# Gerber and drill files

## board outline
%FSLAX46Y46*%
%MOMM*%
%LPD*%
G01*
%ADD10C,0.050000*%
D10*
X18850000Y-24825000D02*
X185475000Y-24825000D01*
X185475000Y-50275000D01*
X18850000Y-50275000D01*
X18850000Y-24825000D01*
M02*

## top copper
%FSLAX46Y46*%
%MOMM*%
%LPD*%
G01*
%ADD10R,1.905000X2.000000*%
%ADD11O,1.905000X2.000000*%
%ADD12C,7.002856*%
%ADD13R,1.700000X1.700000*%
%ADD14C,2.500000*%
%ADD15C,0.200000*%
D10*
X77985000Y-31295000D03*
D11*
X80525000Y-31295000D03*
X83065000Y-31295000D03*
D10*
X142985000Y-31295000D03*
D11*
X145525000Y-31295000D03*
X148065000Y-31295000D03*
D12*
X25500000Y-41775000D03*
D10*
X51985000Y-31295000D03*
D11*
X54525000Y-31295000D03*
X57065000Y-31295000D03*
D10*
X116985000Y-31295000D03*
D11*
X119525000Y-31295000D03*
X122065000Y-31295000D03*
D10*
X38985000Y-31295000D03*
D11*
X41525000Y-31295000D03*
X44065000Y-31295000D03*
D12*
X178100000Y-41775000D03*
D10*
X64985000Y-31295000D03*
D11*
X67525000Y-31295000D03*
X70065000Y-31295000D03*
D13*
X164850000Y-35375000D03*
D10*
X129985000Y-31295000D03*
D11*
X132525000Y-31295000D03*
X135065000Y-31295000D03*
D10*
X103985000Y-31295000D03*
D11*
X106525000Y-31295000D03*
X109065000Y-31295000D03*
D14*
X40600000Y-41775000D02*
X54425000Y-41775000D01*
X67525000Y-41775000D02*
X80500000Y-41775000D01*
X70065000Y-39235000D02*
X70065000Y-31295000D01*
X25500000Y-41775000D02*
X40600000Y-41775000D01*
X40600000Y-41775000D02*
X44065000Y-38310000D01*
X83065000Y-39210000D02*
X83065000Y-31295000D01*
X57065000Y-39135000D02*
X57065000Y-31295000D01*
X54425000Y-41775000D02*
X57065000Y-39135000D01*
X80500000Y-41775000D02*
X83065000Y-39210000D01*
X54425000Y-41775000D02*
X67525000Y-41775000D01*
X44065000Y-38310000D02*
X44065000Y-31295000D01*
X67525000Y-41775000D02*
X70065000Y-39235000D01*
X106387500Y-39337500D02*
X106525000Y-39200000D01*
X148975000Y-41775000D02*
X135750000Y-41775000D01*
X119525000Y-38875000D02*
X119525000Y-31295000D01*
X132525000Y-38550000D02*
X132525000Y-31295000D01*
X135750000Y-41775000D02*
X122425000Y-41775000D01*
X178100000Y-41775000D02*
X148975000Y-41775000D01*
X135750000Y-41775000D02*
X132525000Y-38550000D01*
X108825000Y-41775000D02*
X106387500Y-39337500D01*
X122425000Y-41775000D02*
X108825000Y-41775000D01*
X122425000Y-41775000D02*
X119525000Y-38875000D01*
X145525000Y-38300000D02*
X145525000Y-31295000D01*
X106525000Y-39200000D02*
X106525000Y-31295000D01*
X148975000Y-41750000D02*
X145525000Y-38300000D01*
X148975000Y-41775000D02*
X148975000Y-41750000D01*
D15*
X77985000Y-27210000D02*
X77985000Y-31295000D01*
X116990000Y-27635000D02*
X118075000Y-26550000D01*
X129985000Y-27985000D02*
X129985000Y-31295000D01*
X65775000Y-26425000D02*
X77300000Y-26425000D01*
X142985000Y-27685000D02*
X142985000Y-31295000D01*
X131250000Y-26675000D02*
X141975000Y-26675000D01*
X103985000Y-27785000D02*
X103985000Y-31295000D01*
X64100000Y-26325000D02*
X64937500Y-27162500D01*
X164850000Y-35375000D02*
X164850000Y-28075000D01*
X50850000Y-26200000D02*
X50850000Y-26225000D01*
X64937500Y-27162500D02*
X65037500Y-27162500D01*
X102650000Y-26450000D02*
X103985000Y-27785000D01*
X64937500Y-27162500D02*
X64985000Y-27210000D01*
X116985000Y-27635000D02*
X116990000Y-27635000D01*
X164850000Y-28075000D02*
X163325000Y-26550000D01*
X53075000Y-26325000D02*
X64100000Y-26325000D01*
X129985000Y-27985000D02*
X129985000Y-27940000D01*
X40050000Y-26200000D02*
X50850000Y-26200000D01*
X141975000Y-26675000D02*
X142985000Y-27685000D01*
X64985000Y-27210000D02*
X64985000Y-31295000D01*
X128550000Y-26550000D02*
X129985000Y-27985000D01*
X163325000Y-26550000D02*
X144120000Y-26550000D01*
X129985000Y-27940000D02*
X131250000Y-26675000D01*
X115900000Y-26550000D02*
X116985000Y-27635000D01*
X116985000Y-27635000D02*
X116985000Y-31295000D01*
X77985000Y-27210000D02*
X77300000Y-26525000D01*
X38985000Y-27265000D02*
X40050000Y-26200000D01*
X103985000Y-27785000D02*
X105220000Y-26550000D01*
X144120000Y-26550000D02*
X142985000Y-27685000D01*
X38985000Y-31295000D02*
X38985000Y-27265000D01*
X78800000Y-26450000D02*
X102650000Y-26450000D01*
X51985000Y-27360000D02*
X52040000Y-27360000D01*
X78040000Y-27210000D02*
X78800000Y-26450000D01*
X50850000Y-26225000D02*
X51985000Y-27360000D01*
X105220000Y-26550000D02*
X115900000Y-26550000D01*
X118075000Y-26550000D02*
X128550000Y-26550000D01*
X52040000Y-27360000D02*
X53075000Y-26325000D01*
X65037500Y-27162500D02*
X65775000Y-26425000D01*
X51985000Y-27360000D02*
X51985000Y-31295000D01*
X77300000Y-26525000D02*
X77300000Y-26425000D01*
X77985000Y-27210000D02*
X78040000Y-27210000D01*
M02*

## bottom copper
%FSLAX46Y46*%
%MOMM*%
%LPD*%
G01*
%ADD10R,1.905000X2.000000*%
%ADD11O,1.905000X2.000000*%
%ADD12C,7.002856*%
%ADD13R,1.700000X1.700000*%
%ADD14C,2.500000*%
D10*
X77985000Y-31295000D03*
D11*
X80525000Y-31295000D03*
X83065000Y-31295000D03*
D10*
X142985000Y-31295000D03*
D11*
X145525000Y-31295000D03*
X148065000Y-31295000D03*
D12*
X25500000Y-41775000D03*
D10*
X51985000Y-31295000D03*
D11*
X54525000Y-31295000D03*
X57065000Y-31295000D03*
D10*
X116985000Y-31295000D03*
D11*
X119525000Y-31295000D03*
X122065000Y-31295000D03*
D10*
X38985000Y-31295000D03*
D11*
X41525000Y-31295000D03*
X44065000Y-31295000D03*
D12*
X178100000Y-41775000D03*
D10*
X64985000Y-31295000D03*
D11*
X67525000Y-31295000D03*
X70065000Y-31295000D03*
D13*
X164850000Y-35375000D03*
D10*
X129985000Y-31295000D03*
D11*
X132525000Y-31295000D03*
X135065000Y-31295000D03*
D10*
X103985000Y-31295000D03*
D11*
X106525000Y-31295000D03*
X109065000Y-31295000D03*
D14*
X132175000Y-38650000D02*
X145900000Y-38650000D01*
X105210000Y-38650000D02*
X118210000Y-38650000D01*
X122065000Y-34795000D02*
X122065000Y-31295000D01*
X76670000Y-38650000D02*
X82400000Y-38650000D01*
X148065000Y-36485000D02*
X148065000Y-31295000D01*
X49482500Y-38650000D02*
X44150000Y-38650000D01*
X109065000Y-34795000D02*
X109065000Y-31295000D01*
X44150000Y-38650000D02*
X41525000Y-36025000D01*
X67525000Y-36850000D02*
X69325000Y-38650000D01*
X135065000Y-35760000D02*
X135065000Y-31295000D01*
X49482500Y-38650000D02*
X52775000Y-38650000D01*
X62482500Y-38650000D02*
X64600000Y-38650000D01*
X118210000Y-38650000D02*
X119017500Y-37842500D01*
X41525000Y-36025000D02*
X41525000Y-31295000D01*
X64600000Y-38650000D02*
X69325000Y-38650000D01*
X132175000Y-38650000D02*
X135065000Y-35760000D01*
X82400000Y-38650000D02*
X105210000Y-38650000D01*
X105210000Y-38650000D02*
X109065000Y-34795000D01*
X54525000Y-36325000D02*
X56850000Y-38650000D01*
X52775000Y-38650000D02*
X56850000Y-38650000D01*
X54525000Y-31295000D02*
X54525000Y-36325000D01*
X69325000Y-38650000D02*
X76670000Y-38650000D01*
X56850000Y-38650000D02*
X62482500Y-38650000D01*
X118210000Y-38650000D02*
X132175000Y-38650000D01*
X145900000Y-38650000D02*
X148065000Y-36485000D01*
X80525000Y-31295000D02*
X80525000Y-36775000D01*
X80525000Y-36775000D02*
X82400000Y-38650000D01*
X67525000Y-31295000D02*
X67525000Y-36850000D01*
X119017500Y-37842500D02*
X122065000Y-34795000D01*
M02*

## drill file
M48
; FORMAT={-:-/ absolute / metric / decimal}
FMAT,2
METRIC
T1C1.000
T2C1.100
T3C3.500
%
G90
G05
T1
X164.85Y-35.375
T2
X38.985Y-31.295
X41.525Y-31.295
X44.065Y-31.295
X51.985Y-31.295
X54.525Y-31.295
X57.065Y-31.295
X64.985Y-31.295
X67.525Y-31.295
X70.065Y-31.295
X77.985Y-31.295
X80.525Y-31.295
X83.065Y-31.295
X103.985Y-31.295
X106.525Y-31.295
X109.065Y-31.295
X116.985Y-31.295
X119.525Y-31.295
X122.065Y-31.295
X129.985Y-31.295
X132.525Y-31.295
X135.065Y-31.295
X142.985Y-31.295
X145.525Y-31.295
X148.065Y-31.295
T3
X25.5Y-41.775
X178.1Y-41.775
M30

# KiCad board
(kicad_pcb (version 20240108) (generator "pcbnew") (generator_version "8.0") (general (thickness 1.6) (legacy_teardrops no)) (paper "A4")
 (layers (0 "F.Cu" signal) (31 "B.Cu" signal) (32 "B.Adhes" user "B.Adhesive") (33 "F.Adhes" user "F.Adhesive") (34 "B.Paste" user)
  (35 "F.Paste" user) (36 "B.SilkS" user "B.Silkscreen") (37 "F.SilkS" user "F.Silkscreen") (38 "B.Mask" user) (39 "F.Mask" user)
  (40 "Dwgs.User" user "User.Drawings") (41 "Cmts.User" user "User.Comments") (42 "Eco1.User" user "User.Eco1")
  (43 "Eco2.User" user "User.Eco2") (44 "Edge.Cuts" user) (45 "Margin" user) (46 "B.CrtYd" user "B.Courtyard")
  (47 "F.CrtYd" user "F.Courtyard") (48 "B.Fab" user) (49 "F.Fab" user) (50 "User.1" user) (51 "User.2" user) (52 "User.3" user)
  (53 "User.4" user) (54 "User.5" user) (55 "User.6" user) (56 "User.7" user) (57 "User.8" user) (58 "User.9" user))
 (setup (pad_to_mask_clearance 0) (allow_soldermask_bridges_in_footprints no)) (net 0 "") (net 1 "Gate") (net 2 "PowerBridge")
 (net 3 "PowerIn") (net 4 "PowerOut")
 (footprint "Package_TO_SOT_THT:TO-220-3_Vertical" (layer "F.Cu") (at 77.985 31.295)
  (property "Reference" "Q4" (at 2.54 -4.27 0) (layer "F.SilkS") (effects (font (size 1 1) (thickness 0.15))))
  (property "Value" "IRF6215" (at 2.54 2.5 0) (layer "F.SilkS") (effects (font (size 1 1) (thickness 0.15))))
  (pad "1" thru_hole rect (at 0 0) (size 1.905 2) (drill 1.1) (layers "*.Cu" "*.Mask") (remove_unused_layers no) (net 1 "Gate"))
  (pad "2" thru_hole oval (at 2.54 0) (size 1.905 2) (drill 1.1) (layers "*.Cu" "*.Mask") (remove_unused_layers no) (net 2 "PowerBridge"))
  (pad "3" thru_hole oval (at 5.08 0) (size 1.905 2) (drill 1.1) (layers "*.Cu" "*.Mask") (remove_unused_layers no) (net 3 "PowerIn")))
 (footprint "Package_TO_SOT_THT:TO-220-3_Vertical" (layer "F.Cu") (at 142.985 31.295)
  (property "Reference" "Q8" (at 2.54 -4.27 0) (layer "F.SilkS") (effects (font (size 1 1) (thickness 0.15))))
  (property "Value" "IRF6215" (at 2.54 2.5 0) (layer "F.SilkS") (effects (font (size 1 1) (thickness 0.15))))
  (pad "1" thru_hole rect (at 0 0) (size 1.905 2) (drill 1.1) (layers "*.Cu" "*.Mask") (remove_unused_layers no) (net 1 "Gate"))
  (pad "2" thru_hole oval (at 2.54 0) (size 1.905 2) (drill 1.1) (layers "*.Cu" "*.Mask") (remove_unused_layers no) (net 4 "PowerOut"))
  (pad "3" thru_hole oval (at 5.08 0) (size 1.905 2) (drill 1.1) (layers "*.Cu" "*.Mask") (remove_unused_layers no) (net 2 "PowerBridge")))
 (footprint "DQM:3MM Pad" (layer "F.Cu") (at 25.5 41.775)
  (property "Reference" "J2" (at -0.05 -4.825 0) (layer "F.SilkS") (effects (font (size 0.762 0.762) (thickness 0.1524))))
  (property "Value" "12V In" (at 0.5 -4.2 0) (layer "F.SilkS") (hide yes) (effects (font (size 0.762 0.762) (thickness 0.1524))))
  (pad "1" thru_hole circle (at 0 0) (size 7.002856 7.002856) (drill 3.5) (layers "*.Cu" "*.Mask") (remove_unused_layers no)
   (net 3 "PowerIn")))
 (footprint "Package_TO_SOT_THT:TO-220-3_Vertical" (layer "F.Cu") (at 51.985 31.295)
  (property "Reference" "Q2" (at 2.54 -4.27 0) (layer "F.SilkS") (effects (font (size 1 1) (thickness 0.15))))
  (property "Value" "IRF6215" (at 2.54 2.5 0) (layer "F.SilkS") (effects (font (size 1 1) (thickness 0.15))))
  (pad "1" thru_hole rect (at 0 0) (size 1.905 2) (drill 1.1) (layers "*.Cu" "*.Mask") (remove_unused_layers no) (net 1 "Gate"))
  (pad "2" thru_hole oval (at 2.54 0) (size 1.905 2) (drill 1.1) (layers "*.Cu" "*.Mask") (remove_unused_layers no) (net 2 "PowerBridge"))
  (pad "3" thru_hole oval (at 5.08 0) (size 1.905 2) (drill 1.1) (layers "*.Cu" "*.Mask") (remove_unused_layers no) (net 3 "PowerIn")))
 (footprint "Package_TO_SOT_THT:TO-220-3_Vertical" (layer "F.Cu") (at 116.985 31.295)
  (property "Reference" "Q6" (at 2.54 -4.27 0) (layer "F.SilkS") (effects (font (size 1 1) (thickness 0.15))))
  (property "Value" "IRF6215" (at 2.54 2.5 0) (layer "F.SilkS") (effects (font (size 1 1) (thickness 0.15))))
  (pad "1" thru_hole rect (at 0 0) (size 1.905 2) (drill 1.1) (layers "*.Cu" "*.Mask") (remove_unused_layers no) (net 1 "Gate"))
  (pad "2" thru_hole oval (at 2.54 0) (size 1.905 2) (drill 1.1) (layers "*.Cu" "*.Mask") (remove_unused_layers no) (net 4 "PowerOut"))
  (pad "3" thru_hole oval (at 5.08 0) (size 1.905 2) (drill 1.1) (layers "*.Cu" "*.Mask") (remove_unused_layers no) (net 2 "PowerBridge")))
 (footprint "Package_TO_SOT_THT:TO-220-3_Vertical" (layer "F.Cu") (at 38.985 31.295)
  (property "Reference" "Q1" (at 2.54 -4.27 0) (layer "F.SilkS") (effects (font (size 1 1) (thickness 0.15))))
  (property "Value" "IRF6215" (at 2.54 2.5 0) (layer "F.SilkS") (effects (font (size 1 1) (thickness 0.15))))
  (pad "1" thru_hole rect (at 0 0) (size 1.905 2) (drill 1.1) (layers "*.Cu" "*.Mask") (remove_unused_layers no) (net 1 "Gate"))
  (pad "2" thru_hole oval (at 2.54 0) (size 1.905 2) (drill 1.1) (layers "*.Cu" "*.Mask") (remove_unused_layers no) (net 2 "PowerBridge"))
  (pad "3" thru_hole oval (at 5.08 0) (size 1.905 2) (drill 1.1) (layers "*.Cu" "*.Mask") (remove_unused_layers no) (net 3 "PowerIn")))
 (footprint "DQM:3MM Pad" (layer "F.Cu") (at 178.1 41.775)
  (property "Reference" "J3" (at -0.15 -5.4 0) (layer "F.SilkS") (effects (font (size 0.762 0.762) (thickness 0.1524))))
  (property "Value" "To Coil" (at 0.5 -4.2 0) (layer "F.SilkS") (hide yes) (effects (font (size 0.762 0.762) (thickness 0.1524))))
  (pad "1" thru_hole circle (at 0 0) (size 7.002856 7.002856) (drill 3.5) (layers "*.Cu" "*.Mask") (remove_unused_layers no)
   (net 4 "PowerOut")))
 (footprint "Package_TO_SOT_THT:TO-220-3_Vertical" (layer "F.Cu") (at 64.985 31.295)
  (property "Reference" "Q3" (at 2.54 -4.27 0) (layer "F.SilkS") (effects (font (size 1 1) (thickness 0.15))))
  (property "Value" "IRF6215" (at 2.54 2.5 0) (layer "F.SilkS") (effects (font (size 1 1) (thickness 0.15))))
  (pad "1" thru_hole rect (at 0 0) (size 1.905 2) (drill 1.1) (layers "*.Cu" "*.Mask") (remove_unused_layers no) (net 1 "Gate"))
  (pad "2" thru_hole oval (at 2.54 0) (size 1.905 2) (drill 1.1) (layers "*.Cu" "*.Mask") (remove_unused_layers no) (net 2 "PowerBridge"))
  (pad "3" thru_hole oval (at 5.08 0) (size 1.905 2) (drill 1.1) (layers "*.Cu" "*.Mask") (remove_unused_layers no) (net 3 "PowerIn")))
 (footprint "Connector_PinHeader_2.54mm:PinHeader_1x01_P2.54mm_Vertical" (layer "F.Cu") (at 164.85 35.375)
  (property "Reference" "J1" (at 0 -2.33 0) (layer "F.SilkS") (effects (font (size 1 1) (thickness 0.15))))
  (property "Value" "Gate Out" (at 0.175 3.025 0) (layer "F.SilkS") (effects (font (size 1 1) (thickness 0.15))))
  (pad "1" thru_hole rect (at 0 0) (size 1.7 1.7) (drill 1) (layers "*.Cu" "*.Mask") (remove_unused_layers no) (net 1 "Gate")))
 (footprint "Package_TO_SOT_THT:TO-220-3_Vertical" (layer "F.Cu") (at 129.985 31.295)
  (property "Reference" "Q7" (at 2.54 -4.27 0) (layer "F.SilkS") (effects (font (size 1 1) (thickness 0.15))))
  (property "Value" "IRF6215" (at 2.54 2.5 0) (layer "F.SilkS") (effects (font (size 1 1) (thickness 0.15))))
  (pad "1" thru_hole rect (at 0 0) (size 1.905 2) (drill 1.1) (layers "*.Cu" "*.Mask") (remove_unused_layers no) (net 1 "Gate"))
  (pad "2" thru_hole oval (at 2.54 0) (size 1.905 2) (drill 1.1) (layers "*.Cu" "*.Mask") (remove_unused_layers no) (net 4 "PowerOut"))
  (pad "3" thru_hole oval (at 5.08 0) (size 1.905 2) (drill 1.1) (layers "*.Cu" "*.Mask") (remove_unused_layers no) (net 2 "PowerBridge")))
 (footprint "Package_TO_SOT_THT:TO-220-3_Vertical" (layer "F.Cu") (at 103.985 31.295)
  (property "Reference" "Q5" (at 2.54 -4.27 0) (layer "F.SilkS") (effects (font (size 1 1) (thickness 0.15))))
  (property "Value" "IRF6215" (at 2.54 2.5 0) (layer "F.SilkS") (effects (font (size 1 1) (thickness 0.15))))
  (pad "1" thru_hole rect (at 0 0) (size 1.905 2) (drill 1.1) (layers "*.Cu" "*.Mask") (remove_unused_layers no) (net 1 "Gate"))
  (pad "2" thru_hole oval (at 2.54 0) (size 1.905 2) (drill 1.1) (layers "*.Cu" "*.Mask") (remove_unused_layers no) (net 4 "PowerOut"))
  (pad "3" thru_hole oval (at 5.08 0) (size 1.905 2) (drill 1.1) (layers "*.Cu" "*.Mask") (remove_unused_layers no) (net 2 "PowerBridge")))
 (gr_rect (start 18.85 24.825) (end 185.475 50.275) (stroke (width 0.05) (type default)) (fill none) (layer "Edge.Cuts"))
 (segment (start 40.6 41.775) (end 54.425 41.775) (width 2.5) (layer "F.Cu") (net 3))
 (segment (start 67.525 41.775) (end 80.5 41.775) (width 2.5) (layer "F.Cu") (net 3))
 (segment (start 70.065 39.235) (end 70.065 31.295) (width 2.5) (layer "F.Cu") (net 3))
 (segment (start 25.5 41.775) (end 40.6 41.775) (width 2.5) (layer "F.Cu") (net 3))
 (segment (start 40.6 41.775) (end 44.065 38.31) (width 2.5) (layer "F.Cu") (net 3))
 (segment (start 83.065 39.21) (end 83.065 31.295) (width 2.5) (layer "F.Cu") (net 3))
 (segment (start 57.065 39.135) (end 57.065 31.295) (width 2.5) (layer "F.Cu") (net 3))
 (segment (start 54.425 41.775) (end 57.065 39.135) (width 2.5) (layer "F.Cu") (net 3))
 (segment (start 80.5 41.775) (end 83.065 39.21) (width 2.5) (layer "F.Cu") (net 3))
 (segment (start 54.425 41.775) (end 67.525 41.775) (width 2.5) (layer "F.Cu") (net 3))
 (segment (start 44.065 38.31) (end 44.065 31.295) (width 2.5) (layer "F.Cu") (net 3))
 (segment (start 67.525 41.775) (end 70.065 39.235) (width 2.5) (layer "F.Cu") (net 3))
 (segment (start 106.3875 39.3375) (end 106.525 39.2) (width 2.5) (layer "F.Cu") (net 4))
 (segment (start 148.975 41.775) (end 135.75 41.775) (width 2.5) (layer "F.Cu") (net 4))
 (segment (start 119.525 38.875) (end 119.525 31.295) (width 2.5) (layer "F.Cu") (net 4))
 (segment (start 132.525 38.55) (end 132.525 31.295) (width 2.5) (layer "F.Cu") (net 4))
 (segment (start 135.75 41.775) (end 122.425 41.775) (width 2.5) (layer "F.Cu") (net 4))
 (segment (start 178.1 41.775) (end 148.975 41.775) (width 2.5) (layer "F.Cu") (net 4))
 (segment (start 135.75 41.775) (end 132.525 38.55) (width 2.5) (layer "F.Cu") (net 4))
 (segment (start 108.825 41.775) (end 106.3875 39.3375) (width 2.5) (layer "F.Cu") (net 4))
 (segment (start 122.425 41.775) (end 108.825 41.775) (width 2.5) (layer "F.Cu") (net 4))
 (segment (start 122.425 41.775) (end 119.525 38.875) (width 2.5) (layer "F.Cu") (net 4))
 (segment (start 145.525 38.3) (end 145.525 31.295) (width 2.5) (layer "F.Cu") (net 4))
 (segment (start 106.525 39.2) (end 106.525 31.295) (width 2.5) (layer "F.Cu") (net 4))
 (segment (start 148.975 41.75) (end 145.525 38.3) (width 2.5) (layer "F.Cu") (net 4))
 (segment (start 148.975 41.775) (end 148.975 41.75) (width 2.5) (layer "F.Cu") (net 4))
 (segment (start 77.985 27.21) (end 77.985 31.295) (width 0.2) (layer "F.Cu") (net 1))
 (segment (start 116.99 27.635) (end 118.075 26.55) (width 0.2) (layer "F.Cu") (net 1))
 (segment (start 129.985 27.985) (end 129.985 31.295) (width 0.2) (layer "F.Cu") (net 1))
 (segment (start 65.775 26.425) (end 77.3 26.425) (width 0.2) (layer "F.Cu") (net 1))
 (segment (start 142.985 27.685) (end 142.985 31.295) (width 0.2) (layer "F.Cu") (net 1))
 (segment (start 131.25 26.675) (end 141.975 26.675) (width 0.2) (layer "F.Cu") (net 1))
 (segment (start 103.985 27.785) (end 103.985 31.295) (width 0.2) (layer "F.Cu") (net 1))
 (segment (start 64.1 26.325) (end 64.9375 27.1625) (width 0.2) (layer "F.Cu") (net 1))
 (segment (start 164.85 35.375) (end 164.85 28.075) (width 0.2) (layer "F.Cu") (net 1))
 (segment (start 50.85 26.2) (end 50.85 26.225) (width 0.2) (layer "F.Cu") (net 1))
 (segment (start 64.9375 27.1625) (end 65.0375 27.1625) (width 0.2) (layer "F.Cu") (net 1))
 (segment (start 102.65 26.45) (end 103.985 27.785) (width 0.2) (layer "F.Cu") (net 1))
 (segment (start 64.9375 27.1625) (end 64.985 27.21) (width 0.2) (layer "F.Cu") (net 1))
 (segment (start 116.985 27.635) (end 116.99 27.635) (width 0.2) (layer "F.Cu") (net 1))
 (segment (start 164.85 28.075) (end 163.325 26.55) (width 0.2) (layer "F.Cu") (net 1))
 (segment (start 53.075 26.325) (end 64.1 26.325) (width 0.2) (layer "F.Cu") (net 1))
 (segment (start 129.985 27.985) (end 129.985 27.94) (width 0.2) (layer "F.Cu") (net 1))
 (segment (start 40.05 26.2) (end 50.85 26.2) (width 0.2) (layer "F.Cu") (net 1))
 (segment (start 141.975 26.675) (end 142.985 27.685) (width 0.2) (layer "F.Cu") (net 1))
 (segment (start 64.985 27.21) (end 64.985 31.295) (width 0.2) (layer "F.Cu") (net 1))
 (segment (start 128.55 26.55) (end 129.985 27.985) (width 0.2) (layer "F.Cu") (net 1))
 (segment (start 163.325 26.55) (end 144.12 26.55) (width 0.2) (layer "F.Cu") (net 1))
 (segment (start 129.985 27.94) (end 131.25 26.675) (width 0.2) (layer "F.Cu") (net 1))
 (segment (start 115.9 26.55) (end 116.985 27.635) (width 0.2) (layer "F.Cu") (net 1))
 (segment (start 116.985 27.635) (end 116.985 31.295) (width 0.2) (layer "F.Cu") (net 1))
 (segment (start 77.985 27.21) (end 77.3 26.525) (width 0.2) (layer "F.Cu") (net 1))
 (segment (start 38.985 27.265) (end 40.05 26.2) (width 0.2) (layer "F.Cu") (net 1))
 (segment (start 103.985 27.785) (end 105.22 26.55) (width 0.2) (layer "F.Cu") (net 1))
 (segment (start 144.12 26.55) (end 142.985 27.685) (width 0.2) (layer "F.Cu") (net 1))
 (segment (start 38.985 31.295) (end 38.985 27.265) (width 0.2) (layer "F.Cu") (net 1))
 (segment (start 78.8 26.45) (end 102.65 26.45) (width 0.2) (layer "F.Cu") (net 1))
 (segment (start 51.985 27.36) (end 52.04 27.36) (width 0.2) (layer "F.Cu") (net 1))
 (segment (start 78.04 27.21) (end 78.8 26.45) (width 0.2) (layer "F.Cu") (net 1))
 (segment (start 50.85 26.225) (end 51.985 27.36) (width 0.2) (layer "F.Cu") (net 1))
 (segment (start 105.22 26.55) (end 115.9 26.55) (width 0.2) (layer "F.Cu") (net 1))
 (segment (start 118.075 26.55) (end 128.55 26.55) (width 0.2) (layer "F.Cu") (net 1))
 (segment (start 52.04 27.36) (end 53.075 26.325) (width 0.2) (layer "F.Cu") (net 1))
 (segment (start 65.0375 27.1625) (end 65.775 26.425) (width 0.2) (layer "F.Cu") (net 1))
 (segment (start 51.985 27.36) (end 51.985 31.295) (width 0.2) (layer "F.Cu") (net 1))
 (segment (start 77.3 26.525) (end 77.3 26.425) (width 0.2) (layer "F.Cu") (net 1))
 (segment (start 77.985 27.21) (end 78.04 27.21) (width 0.2) (layer "F.Cu") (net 1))
 (segment (start 132.175 38.65) (end 145.9 38.65) (width 2.5) (layer "B.Cu") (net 2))
 (segment (start 105.21 38.65) (end 118.21 38.65) (width 2.5) (layer "B.Cu") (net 2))
 (segment (start 122.065 34.795) (end 122.065 31.295) (width 2.5) (layer "B.Cu") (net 2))
 (segment (start 76.67 38.65) (end 82.4 38.65) (width 2.5) (layer "B.Cu") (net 2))
 (segment (start 148.065 36.485) (end 148.065 31.295) (width 2.5) (layer "B.Cu") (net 2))
 (segment (start 49.4825 38.65) (end 44.15 38.65) (width 2.5) (layer "B.Cu") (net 2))
 (segment (start 109.065 34.795) (end 109.065 31.295) (width 2.5) (layer "B.Cu") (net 2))
 (segment (start 44.15 38.65) (end 41.525 36.025) (width 2.5) (layer "B.Cu") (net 2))
 (segment (start 67.525 36.85) (end 69.325 38.65) (width 2.5) (layer "B.Cu") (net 2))
 (segment (start 135.065 35.76) (end 135.065 31.295) (width 2.5) (layer "B.Cu") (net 2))
 (segment (start 49.4825 38.65) (end 52.775 38.65) (width 2.5) (layer "B.Cu") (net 2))
 (segment (start 62.4825 38.65) (end 64.6 38.65) (width 2.5) (layer "B.Cu") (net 2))
 (segment (start 118.21 38.65) (end 119.0175 37.8425) (width 2.5) (layer "B.Cu") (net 2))
 (segment (start 41.525 36.025) (end 41.525 31.295) (width 2.5) (layer "B.Cu") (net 2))
 (segment (start 64.6 38.65) (end 69.325 38.65) (width 2.5) (layer "B.Cu") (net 2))
 (segment (start 132.175 38.65) (end 135.065 35.76) (width 2.5) (layer "B.Cu") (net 2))
 (segment (start 82.4 38.65) (end 105.21 38.65) (width 2.5) (layer "B.Cu") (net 2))
 (segment (start 105.21 38.65) (end 109.065 34.795) (width 2.5) (layer "B.Cu") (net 2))
 (segment (start 54.525 36.325) (end 56.85 38.65) (width 2.5) (layer "B.Cu") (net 2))
 (segment (start 52.775 38.65) (end 56.85 38.65) (width 2.5) (layer "B.Cu") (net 2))
 (segment (start 54.525 31.295) (end 54.525 36.325) (width 2.5) (layer "B.Cu") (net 2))
 (segment (start 69.325 38.65) (end 76.67 38.65) (width 2.5) (layer "B.Cu") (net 2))
 (segment (start 56.85 38.65) (end 62.4825 38.65) (width 2.5) (layer "B.Cu") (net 2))
 (segment (start 118.21 38.65) (end 132.175 38.65) (width 2.5) (layer "B.Cu") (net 2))
 (segment (start 145.9 38.65) (end 148.065 36.485) (width 2.5) (layer "B.Cu") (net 2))
 (segment (start 80.525 31.295) (end 80.525 36.775) (width 2.5) (layer "B.Cu") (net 2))
 (segment (start 80.525 36.775) (end 82.4 38.65) (width 2.5) (layer "B.Cu") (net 2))
 (segment (start 67.525 31.295) (end 67.525 36.85) (width 2.5) (layer "B.Cu") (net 2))
 (segment (start 119.0175 37.8425) (end 122.065 34.795) (width 2.5) (layer "B.Cu") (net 2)))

